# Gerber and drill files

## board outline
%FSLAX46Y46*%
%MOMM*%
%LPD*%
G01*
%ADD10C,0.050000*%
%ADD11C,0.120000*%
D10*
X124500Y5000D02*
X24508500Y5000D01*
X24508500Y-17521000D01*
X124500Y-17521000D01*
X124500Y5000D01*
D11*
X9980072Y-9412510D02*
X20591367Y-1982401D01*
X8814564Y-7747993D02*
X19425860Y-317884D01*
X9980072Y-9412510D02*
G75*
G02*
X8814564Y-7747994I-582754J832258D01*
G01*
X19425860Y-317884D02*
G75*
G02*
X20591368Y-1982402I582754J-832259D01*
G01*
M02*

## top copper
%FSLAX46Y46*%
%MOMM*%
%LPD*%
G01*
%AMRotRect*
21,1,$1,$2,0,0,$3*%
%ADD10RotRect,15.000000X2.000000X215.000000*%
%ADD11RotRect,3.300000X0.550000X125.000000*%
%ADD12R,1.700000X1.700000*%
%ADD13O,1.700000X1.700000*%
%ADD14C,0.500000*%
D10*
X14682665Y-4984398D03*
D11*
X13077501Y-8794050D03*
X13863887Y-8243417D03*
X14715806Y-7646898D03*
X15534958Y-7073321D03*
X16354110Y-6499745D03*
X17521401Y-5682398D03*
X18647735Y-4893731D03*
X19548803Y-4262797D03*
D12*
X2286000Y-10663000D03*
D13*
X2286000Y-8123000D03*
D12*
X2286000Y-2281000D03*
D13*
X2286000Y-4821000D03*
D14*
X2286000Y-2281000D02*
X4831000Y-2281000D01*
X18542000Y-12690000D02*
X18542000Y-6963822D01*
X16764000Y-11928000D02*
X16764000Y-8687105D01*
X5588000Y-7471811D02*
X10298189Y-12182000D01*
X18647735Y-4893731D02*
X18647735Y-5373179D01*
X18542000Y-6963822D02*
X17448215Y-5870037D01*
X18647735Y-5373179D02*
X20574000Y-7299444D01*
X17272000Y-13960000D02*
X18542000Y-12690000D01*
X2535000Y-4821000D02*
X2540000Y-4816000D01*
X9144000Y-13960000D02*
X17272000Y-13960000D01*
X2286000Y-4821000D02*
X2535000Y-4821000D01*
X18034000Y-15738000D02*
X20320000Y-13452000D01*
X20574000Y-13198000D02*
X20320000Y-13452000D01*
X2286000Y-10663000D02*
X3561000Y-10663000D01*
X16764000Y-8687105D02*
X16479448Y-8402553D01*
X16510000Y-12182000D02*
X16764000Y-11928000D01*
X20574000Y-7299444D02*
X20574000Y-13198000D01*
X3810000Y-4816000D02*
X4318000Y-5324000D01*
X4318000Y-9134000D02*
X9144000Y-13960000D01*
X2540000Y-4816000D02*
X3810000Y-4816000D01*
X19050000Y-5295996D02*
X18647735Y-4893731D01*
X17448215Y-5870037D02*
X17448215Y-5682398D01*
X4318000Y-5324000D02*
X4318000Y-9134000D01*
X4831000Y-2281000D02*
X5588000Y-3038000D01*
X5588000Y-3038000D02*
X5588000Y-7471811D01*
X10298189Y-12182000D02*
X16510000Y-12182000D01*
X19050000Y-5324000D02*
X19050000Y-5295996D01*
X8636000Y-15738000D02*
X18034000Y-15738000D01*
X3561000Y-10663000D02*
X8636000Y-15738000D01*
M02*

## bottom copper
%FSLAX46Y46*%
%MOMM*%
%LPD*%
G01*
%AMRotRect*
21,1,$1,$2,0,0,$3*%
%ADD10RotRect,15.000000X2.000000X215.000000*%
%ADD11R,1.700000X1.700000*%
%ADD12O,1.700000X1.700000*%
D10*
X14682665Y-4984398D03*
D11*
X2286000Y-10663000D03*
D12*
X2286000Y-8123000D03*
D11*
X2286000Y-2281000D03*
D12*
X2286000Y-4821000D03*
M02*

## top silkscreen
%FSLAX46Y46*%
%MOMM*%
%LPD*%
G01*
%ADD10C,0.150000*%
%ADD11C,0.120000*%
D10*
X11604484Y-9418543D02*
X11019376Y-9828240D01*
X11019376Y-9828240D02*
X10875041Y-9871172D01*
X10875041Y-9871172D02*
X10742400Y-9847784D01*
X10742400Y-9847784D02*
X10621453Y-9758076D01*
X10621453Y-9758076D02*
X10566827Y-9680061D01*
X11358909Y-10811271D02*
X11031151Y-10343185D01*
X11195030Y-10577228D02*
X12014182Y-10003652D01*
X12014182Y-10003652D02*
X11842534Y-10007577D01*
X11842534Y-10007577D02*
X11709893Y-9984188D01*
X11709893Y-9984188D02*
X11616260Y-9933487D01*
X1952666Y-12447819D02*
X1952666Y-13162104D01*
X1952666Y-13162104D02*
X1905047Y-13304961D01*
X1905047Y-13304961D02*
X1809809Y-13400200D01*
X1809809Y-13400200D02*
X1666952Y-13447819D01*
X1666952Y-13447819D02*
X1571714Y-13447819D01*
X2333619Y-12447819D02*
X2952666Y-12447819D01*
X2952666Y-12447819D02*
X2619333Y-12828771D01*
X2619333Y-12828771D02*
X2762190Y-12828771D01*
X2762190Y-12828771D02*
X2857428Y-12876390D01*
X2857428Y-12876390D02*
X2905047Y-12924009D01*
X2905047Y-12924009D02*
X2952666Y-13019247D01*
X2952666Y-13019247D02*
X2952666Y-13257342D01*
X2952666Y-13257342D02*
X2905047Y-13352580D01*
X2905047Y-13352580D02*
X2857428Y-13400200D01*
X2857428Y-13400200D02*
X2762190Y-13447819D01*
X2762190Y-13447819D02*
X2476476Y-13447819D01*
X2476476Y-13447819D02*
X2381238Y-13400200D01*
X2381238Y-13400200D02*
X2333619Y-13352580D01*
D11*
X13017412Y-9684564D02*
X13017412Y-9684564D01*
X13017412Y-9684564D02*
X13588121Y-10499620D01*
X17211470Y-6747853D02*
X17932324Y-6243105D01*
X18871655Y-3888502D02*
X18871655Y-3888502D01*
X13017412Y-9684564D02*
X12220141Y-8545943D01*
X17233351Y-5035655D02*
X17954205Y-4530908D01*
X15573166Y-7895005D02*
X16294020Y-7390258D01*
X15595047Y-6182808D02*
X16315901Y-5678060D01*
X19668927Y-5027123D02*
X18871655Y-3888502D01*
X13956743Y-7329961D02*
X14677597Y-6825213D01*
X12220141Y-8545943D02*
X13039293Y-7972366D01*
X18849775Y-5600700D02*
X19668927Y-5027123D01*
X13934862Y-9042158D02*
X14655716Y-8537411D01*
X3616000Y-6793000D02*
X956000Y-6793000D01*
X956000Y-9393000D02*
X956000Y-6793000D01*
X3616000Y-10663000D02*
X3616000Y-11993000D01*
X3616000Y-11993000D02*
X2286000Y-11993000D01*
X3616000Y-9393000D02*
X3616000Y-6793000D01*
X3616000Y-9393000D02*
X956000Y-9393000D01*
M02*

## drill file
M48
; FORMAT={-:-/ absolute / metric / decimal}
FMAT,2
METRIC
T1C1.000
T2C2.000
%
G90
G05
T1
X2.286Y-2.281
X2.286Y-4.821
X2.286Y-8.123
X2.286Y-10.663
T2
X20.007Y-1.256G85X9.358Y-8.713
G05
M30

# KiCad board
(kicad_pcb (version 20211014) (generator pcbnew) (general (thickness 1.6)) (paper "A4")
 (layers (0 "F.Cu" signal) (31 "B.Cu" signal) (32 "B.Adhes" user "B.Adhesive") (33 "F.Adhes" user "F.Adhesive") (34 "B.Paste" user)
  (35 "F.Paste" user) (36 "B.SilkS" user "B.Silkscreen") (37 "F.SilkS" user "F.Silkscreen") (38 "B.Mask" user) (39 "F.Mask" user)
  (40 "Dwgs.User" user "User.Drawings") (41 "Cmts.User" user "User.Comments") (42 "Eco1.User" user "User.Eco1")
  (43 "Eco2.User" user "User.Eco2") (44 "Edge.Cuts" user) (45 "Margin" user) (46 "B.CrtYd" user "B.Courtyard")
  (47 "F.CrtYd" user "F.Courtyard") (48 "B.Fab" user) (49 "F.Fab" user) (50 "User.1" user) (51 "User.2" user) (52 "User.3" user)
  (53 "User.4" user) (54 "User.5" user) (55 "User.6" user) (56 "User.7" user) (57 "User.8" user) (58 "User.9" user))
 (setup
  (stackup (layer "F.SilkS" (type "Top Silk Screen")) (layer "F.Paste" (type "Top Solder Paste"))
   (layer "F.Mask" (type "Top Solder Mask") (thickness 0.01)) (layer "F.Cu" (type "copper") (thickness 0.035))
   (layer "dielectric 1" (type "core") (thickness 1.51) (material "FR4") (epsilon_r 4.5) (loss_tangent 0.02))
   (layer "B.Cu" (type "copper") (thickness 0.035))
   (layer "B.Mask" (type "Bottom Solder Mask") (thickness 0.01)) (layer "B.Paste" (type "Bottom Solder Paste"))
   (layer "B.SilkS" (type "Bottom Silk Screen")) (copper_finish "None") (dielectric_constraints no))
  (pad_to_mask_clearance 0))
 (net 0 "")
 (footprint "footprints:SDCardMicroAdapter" (layer "F.Cu") (at 15.494 7.102 125)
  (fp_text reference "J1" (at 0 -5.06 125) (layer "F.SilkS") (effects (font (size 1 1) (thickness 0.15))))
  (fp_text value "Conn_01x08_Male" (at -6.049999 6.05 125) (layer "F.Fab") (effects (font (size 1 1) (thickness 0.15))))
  (fp_line (start -0.695 -3.51) (end -0.695 -3.51) (layer "F.SilkS") (width 0.12))
  (fp_line (start -0.695 -3.51) (end -1.69 -3.51) (layer "F.SilkS") (width 0.12))
  (fp_line (start -0.695 1.61) (end -0.695 2.49) (layer "F.SilkS") (width 0.12))
  (fp_line (start 0.695 4.61) (end 0.695 4.61) (layer "F.SilkS") (width 0.12))
  (fp_line (start -0.695 -3.51) (end 0.695 -3.51) (layer "F.SilkS") (width 0.12))
  (fp_line (start 0.695 2.61) (end 0.695 3.49) (layer "F.SilkS") (width 0.12))
  (fp_line (start -0.695 -0.39) (end -0.695 0.49) (layer "F.SilkS") (width 0.12))
  (fp_line (start 0.695 0.61) (end 0.695 1.49) (layer "F.SilkS") (width 0.12))
  (fp_line (start -0.695 4.61) (end 0.695 4.61) (layer "F.SilkS") (width 0.12))
  (fp_line (start 0.695 -1.39) (end 0.695 -0.51) (layer "F.SilkS") (width 0.12))
  (fp_line (start 0.695 -3.51) (end 0.695 -2.51) (layer "F.SilkS") (width 0.12))
  (fp_line (start -0.695 3.61) (end -0.695 4.61) (layer "F.SilkS") (width 0.12))
  (fp_line (start -0.695 -2.39) (end -0.695 -1.51) (layer "F.SilkS") (width 0.12))
  (fp_line (start 1.27 -5.842) (end 1.27 7.112) (layer "Edge.Cuts") (width 0.12))
  (fp_line (start 3.302 -5.842) (end 3.302 7.112) (layer "Edge.Cuts") (width 0.12))
  (fp_arc (start 1.27 -5.842) (mid 2.286 -6.858) (end 3.302 -5.842) (layer "Edge.Cuts") (width 0.12))
  (fp_arc (start 3.302 7.112) (mid 2.286 8.128) (end 1.27 7.112) (layer "Edge.Cuts") (width 0.12))
  (pad "" np_thru_hole rect (at 2.200001 0.55 215) (size 15 2) (drill oval 15 2) (layers F&B.Cu *.Mask))
  (pad "1" smd rect (at 0 -2.95 125) (size 3.3 0.55) (layers "F.Cu" "F.Paste" "F.Mask"))
  (pad "2" smd rect (at 0 -1.99 125) (size 3.3 0.55) (layers "F.Cu" "F.Paste" "F.Mask"))
  (pad "3" smd rect (at 0 -0.95 125) (size 3.3 0.55) (layers "F.Cu" "F.Paste" "F.Mask"))
  (pad "4" smd rect (at 0 0.05 125) (size 3.3 0.55) (layers "F.Cu" "F.Paste" "F.Mask"))
  (pad "5" smd rect (at 0 1.05 125) (size 3.3 0.55) (layers "F.Cu" "F.Paste" "F.Mask"))
  (pad "6" smd rect (at 0 2.475 125) (size 3.3 0.55) (layers "F.Cu" "F.Paste" "F.Mask"))
  (pad "7" smd rect (at 0 3.85 125) (size 3.3 0.55) (layers "F.Cu" "F.Paste" "F.Mask"))
  (pad "8" smd rect (at 0 4.95 125) (size 3.3 0.55) (layers "F.Cu" "F.Paste" "F.Mask")))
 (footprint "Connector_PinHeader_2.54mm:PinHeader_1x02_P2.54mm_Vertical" (layer "F.Cu") (at 2.286 10.663 180)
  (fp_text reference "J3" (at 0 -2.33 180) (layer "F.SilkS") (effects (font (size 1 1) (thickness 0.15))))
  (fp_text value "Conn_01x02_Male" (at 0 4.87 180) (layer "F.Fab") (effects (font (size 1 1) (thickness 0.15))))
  (fp_line (start -1.33 3.87) (end 1.33 3.87) (layer "F.SilkS") (width 0.12))
  (fp_line (start 1.33 1.27) (end 1.33 3.87) (layer "F.SilkS") (width 0.12))
  (fp_line (start -1.33 0) (end -1.33 -1.33) (layer "F.SilkS") (width 0.12))
  (fp_line (start -1.33 -1.33) (end 0 -1.33) (layer "F.SilkS") (width 0.12))
  (fp_line (start -1.33 1.27) (end -1.33 3.87) (layer "F.SilkS") (width 0.12))
  (fp_line (start -1.33 1.27) (end 1.33 1.27) (layer "F.SilkS") (width 0.12))
  (pad "1" thru_hole rect (at 0 0 180) (size 1.7 1.7) (drill 1) (layers *.Cu *.Mask))
  (pad "2" thru_hole oval (at 0 2.54 180) (size 1.7 1.7) (drill 1) (layers *.Cu *.Mask)))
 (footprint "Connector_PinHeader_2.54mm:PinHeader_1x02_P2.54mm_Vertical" (layer "B.Cu") (at 2.286 2.281 180)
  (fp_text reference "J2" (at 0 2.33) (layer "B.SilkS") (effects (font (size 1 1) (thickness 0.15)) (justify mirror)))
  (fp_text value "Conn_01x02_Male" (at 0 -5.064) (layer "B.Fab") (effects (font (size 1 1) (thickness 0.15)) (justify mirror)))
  (pad "1" thru_hole rect (at 0 0 180) (size 1.7 1.7) (drill 1) (layers *.Cu *.Mask))
  (pad "2" thru_hole oval (at 0 -2.54 180) (size 1.7 1.7) (drill 1) (layers *.Cu *.Mask)))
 (gr_rect (start 0.1245 -0.005) (end 24.5085 17.521) (layer "Edge.Cuts") (width 0.05) (fill none))
 (segment (start 2.286 2.281) (end 4.831 2.281) (width 0.5) (layer "F.Cu") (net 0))
 (segment (start 18.542 12.69) (end 18.542 6.963822) (width 0.5) (layer "F.Cu") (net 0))
 (segment (start 16.764 11.928) (end 16.764 8.687105) (width 0.5) (layer "F.Cu") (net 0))
 (segment (start 5.588 7.471811) (end 10.298189 12.182) (width 0.5) (layer "F.Cu") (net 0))
 (segment (start 18.647735 4.893731) (end 18.647735 5.373179) (width 0.5) (layer "F.Cu") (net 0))
 (segment (start 18.542 6.963822) (end 17.448215 5.870037) (width 0.5) (layer "F.Cu") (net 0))
 (segment (start 18.647735 5.373179) (end 20.574 7.299444) (width 0.5) (layer "F.Cu") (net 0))
 (segment (start 17.272 13.96) (end 18.542 12.69) (width 0.5) (layer "F.Cu") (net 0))
 (segment (start 2.535 4.821) (end 2.54 4.816) (width 0.5) (layer "F.Cu") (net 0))
 (segment (start 9.144 13.96) (end 17.272 13.96) (width 0.5) (layer "F.Cu") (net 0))
 (segment (start 2.286 4.821) (end 2.535 4.821) (width 0.5) (layer "F.Cu") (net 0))
 (segment (start 18.034 15.738) (end 20.32 13.452) (width 0.5) (layer "F.Cu") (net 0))
 (segment (start 20.574 13.198) (end 20.32 13.452) (width 0.5) (layer "F.Cu") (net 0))
 (segment (start 2.286 10.663) (end 3.561 10.663) (width 0.5) (layer "F.Cu") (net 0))
 (segment (start 16.764 8.687105) (end 16.479448 8.402553) (width 0.5) (layer "F.Cu") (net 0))
 (segment (start 16.51 12.182) (end 16.764 11.928) (width 0.5) (layer "F.Cu") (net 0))
 (segment (start 20.574 7.299444) (end 20.574 13.198) (width 0.5) (layer "F.Cu") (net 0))
 (segment (start 3.81 4.816) (end 4.318 5.324) (width 0.5) (layer "F.Cu") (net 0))
 (segment (start 4.318 9.134) (end 9.144 13.96) (width 0.5) (layer "F.Cu") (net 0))
 (segment (start 2.54 4.816) (end 3.81 4.816) (width 0.5) (layer "F.Cu") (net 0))
 (segment (start 19.05 5.295996) (end 18.647735 4.893731) (width 0.5) (layer "F.Cu") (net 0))
 (segment (start 17.448215 5.870037) (end 17.448215 5.682398) (width 0.5) (layer "F.Cu") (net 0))
 (segment (start 4.318 5.324) (end 4.318 9.134) (width 0.5) (layer "F.Cu") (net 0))
 (segment (start 4.831 2.281) (end 5.588 3.038) (width 0.5) (layer "F.Cu") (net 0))
 (segment (start 5.588 3.038) (end 5.588 7.471811) (width 0.5) (layer "F.Cu") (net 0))
 (segment (start 10.298189 12.182) (end 16.51 12.182) (width 0.5) (layer "F.Cu") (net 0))
 (segment (start 19.05 5.324) (end 19.05 5.295996) (width 0.5) (layer "F.Cu") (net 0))
 (segment (start 8.636 15.738) (end 18.034 15.738) (width 0.5) (layer "F.Cu") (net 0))
 (segment (start 3.561 10.663) (end 8.636 15.738) (width 0.5) (layer "F.Cu") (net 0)))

